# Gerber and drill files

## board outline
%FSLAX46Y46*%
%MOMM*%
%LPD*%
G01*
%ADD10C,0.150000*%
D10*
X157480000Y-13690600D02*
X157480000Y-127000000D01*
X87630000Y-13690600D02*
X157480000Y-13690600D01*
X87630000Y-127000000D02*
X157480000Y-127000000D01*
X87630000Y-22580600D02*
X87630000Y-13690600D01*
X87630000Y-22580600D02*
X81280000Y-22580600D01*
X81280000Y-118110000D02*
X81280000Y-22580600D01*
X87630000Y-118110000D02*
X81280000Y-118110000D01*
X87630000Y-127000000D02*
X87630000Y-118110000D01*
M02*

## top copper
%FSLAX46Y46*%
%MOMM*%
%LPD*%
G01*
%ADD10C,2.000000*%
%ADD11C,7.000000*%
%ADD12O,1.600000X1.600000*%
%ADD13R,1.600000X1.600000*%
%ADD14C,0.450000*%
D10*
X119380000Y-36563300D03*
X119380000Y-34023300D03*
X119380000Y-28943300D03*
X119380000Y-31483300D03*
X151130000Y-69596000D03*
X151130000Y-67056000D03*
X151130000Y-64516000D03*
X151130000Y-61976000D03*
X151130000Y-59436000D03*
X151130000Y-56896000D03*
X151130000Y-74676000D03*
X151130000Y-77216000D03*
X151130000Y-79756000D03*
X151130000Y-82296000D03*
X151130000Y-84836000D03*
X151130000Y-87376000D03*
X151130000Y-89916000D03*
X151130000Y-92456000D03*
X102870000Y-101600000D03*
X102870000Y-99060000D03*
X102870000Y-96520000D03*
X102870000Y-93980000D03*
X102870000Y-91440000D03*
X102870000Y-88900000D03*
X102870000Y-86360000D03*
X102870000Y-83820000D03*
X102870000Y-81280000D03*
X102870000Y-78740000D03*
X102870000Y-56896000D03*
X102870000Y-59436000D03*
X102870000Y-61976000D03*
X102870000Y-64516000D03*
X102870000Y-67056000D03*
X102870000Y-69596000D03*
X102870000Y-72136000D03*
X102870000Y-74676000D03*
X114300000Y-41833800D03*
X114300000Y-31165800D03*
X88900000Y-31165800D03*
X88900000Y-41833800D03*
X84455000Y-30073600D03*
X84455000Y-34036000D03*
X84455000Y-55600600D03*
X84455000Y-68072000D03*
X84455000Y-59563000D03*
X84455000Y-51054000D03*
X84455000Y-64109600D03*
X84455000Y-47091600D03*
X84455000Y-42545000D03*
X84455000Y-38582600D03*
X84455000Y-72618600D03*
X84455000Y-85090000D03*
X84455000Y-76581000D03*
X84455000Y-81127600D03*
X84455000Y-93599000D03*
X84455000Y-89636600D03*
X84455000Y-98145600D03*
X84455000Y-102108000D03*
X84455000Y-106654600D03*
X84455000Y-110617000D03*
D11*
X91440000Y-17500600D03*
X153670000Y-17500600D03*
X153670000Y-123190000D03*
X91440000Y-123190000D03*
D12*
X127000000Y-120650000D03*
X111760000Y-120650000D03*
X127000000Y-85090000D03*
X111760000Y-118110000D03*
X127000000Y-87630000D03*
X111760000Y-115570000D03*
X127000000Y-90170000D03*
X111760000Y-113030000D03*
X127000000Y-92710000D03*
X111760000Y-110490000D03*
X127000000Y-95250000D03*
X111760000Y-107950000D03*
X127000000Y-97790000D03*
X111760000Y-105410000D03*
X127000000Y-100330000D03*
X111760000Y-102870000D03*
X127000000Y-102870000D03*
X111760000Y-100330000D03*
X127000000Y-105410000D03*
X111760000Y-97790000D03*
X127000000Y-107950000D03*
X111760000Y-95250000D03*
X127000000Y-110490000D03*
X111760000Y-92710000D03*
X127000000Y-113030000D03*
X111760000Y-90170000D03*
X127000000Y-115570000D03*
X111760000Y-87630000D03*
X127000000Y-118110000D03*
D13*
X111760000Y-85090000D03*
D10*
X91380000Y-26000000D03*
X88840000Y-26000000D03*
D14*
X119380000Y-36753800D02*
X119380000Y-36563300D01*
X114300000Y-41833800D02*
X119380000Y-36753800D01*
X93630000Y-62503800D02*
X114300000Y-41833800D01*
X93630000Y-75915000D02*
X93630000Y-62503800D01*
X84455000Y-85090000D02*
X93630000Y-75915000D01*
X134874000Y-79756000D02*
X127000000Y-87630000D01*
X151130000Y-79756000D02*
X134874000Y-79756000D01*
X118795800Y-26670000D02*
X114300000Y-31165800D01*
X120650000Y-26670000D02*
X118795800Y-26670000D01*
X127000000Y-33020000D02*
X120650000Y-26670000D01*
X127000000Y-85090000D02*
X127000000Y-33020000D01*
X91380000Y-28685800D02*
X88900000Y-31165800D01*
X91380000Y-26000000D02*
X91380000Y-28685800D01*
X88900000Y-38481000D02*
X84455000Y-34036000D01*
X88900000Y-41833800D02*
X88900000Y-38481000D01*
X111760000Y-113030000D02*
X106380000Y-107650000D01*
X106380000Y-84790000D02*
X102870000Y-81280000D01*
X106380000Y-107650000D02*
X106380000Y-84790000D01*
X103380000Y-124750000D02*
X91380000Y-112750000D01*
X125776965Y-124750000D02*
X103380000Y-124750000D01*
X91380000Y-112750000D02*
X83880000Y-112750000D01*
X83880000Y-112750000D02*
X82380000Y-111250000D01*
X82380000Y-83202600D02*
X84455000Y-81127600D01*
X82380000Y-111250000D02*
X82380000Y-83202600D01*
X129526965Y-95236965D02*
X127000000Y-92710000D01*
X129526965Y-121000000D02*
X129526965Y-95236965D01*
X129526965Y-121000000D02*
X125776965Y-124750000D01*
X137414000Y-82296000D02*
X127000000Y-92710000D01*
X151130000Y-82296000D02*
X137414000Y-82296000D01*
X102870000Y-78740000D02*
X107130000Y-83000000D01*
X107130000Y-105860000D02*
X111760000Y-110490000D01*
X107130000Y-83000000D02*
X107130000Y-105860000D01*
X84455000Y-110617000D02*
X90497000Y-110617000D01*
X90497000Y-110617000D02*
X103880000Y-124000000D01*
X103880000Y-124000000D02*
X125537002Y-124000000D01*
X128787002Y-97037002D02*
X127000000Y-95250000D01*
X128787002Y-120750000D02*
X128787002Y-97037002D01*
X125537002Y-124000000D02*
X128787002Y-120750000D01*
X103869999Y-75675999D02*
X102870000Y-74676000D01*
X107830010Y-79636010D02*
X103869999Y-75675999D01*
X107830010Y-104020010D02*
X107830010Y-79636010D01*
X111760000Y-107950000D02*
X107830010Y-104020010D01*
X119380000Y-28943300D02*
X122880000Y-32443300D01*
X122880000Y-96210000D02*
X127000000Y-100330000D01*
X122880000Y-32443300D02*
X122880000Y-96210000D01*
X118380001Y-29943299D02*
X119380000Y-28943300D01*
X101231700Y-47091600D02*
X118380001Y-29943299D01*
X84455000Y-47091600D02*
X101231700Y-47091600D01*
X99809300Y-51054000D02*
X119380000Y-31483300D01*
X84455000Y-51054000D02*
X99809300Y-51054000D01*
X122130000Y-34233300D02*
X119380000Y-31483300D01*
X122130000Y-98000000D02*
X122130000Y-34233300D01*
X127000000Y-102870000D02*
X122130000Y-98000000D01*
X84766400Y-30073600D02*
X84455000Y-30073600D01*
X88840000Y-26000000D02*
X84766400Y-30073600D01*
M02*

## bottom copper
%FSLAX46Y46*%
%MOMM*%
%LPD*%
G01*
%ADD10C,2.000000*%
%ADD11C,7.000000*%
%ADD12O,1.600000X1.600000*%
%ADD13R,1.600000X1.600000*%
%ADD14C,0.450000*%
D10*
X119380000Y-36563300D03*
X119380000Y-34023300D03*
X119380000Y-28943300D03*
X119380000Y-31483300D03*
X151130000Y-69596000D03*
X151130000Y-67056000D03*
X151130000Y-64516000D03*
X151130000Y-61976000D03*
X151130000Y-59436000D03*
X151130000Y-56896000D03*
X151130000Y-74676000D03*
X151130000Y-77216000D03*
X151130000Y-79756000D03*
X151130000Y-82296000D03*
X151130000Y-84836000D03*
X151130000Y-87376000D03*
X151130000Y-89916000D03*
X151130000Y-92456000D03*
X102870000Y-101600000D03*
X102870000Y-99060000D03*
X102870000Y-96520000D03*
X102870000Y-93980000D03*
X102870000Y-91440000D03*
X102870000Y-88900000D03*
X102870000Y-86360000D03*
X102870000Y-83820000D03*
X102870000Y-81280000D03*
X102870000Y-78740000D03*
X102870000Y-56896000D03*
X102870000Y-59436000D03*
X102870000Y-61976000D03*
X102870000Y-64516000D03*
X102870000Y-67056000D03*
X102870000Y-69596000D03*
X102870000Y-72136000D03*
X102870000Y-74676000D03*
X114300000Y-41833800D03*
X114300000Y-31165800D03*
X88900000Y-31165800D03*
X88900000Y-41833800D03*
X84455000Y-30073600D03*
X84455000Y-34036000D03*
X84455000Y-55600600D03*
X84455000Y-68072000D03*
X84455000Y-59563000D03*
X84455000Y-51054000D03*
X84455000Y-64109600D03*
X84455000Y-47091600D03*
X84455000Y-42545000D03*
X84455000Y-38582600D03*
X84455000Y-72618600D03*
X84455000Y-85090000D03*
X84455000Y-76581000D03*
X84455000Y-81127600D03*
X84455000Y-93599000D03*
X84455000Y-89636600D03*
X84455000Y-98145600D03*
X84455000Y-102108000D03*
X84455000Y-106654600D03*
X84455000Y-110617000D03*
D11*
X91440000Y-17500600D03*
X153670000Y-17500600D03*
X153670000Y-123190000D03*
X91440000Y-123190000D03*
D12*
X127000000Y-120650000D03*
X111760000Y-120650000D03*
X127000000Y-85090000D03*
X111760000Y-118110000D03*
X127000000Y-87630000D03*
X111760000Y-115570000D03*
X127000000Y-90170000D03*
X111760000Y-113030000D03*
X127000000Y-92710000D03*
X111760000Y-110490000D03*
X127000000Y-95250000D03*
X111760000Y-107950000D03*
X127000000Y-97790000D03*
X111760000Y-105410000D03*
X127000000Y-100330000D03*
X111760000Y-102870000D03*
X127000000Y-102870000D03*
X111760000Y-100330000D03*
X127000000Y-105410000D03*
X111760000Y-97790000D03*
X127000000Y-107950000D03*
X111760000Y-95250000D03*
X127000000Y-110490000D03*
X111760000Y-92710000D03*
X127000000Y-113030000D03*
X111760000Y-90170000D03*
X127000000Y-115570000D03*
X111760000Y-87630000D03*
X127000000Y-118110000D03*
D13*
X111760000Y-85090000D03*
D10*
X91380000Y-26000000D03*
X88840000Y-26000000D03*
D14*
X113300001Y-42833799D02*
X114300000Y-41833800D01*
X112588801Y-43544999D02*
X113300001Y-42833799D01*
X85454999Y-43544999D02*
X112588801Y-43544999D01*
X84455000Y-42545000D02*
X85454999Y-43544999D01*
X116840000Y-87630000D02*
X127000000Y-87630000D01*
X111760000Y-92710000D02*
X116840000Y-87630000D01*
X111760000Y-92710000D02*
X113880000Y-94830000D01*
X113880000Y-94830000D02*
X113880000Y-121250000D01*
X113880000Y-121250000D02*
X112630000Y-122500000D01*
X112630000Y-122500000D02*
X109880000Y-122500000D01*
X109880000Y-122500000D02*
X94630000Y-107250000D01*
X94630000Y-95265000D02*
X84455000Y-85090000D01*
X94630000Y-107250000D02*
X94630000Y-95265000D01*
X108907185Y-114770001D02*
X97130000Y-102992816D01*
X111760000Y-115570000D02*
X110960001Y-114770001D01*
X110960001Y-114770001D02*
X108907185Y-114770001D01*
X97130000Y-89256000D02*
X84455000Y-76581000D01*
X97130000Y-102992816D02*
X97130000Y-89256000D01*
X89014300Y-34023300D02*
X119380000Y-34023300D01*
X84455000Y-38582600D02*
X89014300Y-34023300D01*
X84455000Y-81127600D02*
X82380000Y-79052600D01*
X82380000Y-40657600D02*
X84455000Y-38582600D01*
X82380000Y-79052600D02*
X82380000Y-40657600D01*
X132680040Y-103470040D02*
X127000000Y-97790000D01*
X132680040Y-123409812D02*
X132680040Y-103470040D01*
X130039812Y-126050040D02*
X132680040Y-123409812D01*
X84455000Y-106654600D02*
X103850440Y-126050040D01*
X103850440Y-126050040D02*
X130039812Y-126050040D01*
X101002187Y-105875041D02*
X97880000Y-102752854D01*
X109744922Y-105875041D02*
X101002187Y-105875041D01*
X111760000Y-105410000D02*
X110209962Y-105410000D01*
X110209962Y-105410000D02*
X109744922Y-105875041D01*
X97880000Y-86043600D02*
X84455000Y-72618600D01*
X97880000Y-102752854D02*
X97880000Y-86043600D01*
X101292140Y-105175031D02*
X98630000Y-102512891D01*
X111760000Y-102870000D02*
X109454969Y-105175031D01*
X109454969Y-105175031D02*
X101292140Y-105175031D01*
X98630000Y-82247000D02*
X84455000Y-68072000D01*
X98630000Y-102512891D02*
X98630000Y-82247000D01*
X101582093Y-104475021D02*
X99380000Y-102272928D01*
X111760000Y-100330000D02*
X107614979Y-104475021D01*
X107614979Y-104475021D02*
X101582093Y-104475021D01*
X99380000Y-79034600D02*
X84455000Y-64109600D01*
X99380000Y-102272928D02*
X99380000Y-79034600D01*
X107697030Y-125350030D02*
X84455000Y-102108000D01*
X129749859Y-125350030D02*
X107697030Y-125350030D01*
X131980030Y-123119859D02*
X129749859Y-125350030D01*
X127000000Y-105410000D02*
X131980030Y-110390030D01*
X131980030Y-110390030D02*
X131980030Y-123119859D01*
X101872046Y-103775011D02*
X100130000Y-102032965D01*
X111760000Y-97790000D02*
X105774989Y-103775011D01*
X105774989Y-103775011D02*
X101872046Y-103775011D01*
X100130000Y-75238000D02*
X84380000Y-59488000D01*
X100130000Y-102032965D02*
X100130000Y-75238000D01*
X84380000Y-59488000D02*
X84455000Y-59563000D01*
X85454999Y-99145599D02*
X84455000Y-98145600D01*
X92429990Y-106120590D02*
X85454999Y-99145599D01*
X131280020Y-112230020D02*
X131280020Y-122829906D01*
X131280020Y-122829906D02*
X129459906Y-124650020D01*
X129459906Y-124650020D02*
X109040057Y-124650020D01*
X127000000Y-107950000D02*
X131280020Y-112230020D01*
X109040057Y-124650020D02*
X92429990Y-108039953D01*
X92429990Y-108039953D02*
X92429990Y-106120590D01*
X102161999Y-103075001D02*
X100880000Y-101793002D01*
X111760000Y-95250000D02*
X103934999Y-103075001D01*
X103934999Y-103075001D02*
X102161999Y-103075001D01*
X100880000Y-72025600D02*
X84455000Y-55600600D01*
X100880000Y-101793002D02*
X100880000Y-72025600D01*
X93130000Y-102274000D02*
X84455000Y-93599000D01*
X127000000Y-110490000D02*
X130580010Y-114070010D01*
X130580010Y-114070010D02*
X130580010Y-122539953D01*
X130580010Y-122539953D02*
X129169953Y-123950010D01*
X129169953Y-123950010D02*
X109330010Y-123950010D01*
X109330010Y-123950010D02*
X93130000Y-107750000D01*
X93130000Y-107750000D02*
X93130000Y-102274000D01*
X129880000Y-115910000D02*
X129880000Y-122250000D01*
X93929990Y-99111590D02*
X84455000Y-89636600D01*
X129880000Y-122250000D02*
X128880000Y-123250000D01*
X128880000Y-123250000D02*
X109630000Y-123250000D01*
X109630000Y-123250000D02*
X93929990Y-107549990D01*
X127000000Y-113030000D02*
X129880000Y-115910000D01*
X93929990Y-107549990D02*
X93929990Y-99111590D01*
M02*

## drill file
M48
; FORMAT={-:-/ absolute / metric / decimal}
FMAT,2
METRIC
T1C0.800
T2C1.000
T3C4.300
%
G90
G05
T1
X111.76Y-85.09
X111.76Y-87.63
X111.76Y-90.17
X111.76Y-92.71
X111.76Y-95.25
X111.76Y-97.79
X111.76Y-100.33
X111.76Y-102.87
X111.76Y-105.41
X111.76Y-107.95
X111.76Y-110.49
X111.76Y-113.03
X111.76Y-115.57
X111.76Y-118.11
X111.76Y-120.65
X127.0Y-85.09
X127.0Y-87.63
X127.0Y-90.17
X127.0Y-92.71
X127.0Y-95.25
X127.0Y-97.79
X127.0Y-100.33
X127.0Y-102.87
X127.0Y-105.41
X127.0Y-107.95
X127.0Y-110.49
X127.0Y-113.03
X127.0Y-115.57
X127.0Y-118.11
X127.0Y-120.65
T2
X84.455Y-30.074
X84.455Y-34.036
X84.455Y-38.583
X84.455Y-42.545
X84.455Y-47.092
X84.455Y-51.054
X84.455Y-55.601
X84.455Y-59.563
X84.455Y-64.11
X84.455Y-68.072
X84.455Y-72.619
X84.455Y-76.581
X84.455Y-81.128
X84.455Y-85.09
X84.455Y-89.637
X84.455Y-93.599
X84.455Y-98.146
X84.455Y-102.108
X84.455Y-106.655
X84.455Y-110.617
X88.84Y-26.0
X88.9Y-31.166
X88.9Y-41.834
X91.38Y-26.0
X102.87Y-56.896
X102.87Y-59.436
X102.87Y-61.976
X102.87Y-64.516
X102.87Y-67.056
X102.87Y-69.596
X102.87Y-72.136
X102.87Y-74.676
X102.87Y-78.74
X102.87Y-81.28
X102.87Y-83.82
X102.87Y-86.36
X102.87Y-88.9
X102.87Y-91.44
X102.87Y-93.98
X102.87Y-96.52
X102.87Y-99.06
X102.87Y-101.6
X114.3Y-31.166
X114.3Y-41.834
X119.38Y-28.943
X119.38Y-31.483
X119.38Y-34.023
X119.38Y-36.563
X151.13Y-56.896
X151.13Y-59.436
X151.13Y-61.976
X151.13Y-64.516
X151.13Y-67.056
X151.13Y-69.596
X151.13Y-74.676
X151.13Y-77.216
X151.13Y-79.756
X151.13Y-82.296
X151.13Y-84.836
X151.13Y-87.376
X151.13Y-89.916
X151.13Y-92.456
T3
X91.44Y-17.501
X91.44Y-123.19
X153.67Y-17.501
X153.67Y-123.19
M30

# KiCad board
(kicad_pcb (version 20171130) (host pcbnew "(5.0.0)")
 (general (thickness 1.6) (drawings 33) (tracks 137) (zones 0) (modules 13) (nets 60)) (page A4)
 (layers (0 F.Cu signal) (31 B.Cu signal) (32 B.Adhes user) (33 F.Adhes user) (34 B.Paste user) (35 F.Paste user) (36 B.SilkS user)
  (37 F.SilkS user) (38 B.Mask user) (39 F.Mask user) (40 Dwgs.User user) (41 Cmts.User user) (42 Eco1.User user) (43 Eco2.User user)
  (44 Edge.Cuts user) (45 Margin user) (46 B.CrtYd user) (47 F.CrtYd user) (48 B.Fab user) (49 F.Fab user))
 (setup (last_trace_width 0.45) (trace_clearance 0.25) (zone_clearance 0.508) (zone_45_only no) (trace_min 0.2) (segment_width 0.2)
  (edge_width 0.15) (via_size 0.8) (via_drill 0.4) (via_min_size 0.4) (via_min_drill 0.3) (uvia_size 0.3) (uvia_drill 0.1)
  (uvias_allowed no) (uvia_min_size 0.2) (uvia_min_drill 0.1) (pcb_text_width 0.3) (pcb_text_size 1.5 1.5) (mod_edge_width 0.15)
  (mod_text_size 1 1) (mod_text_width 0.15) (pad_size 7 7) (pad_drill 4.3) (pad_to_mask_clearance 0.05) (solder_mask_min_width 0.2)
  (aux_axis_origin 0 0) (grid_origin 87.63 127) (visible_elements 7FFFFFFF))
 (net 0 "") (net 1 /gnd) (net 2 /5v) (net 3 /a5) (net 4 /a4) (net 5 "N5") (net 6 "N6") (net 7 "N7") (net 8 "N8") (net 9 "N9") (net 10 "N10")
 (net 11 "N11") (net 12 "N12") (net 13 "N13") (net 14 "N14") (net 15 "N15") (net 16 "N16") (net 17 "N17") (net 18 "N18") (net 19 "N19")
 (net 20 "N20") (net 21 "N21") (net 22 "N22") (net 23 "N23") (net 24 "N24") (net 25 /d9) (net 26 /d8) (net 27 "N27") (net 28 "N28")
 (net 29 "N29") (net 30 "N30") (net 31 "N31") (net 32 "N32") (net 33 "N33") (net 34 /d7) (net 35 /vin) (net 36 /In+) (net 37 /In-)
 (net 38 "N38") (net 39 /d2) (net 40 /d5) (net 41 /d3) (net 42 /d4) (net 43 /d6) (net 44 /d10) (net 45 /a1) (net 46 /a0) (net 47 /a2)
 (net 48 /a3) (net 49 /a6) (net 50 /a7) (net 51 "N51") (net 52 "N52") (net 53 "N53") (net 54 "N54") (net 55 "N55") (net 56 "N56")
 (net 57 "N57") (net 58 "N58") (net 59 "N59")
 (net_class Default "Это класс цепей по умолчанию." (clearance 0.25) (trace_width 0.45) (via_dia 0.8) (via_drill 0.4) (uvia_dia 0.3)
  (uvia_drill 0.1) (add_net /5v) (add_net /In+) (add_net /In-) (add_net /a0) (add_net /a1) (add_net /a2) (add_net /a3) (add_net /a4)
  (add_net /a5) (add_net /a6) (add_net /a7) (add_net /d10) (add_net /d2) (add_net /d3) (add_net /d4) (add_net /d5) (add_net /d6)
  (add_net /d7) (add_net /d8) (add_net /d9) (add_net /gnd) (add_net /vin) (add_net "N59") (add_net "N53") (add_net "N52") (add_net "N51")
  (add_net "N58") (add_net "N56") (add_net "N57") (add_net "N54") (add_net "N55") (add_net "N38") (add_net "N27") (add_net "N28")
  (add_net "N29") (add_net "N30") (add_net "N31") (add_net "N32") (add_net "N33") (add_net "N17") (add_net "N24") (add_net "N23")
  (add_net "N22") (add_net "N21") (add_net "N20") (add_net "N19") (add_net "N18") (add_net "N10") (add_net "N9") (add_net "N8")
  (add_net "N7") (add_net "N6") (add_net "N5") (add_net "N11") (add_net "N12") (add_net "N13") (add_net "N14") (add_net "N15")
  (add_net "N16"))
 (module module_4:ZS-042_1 (layer F.Cu) (at 119.38 36.5633)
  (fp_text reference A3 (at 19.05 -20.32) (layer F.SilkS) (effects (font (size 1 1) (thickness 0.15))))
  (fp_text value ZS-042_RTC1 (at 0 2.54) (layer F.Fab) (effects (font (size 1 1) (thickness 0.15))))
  (pad 6 thru_hole circle (at 0 0) (size 2 2) (drill 1) (layers *.Cu *.Mask) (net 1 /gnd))
  (pad 5 thru_hole circle (at 0 -2.54) (size 2 2) (drill 1) (layers *.Cu *.Mask) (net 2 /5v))
  (pad 3 thru_hole circle (at 0 -7.62) (size 2 2) (drill 1) (layers *.Cu *.Mask) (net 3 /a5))
  (pad 4 thru_hole circle (at 0 -5.08) (size 2 2) (drill 1) (layers *.Cu *.Mask) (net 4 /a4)))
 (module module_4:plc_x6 (layer F.Cu) (at 151.13 69.596)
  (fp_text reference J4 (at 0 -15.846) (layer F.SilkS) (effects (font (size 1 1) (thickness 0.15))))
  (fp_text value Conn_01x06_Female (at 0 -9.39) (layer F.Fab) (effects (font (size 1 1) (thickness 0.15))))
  (pad 6 thru_hole circle (at 0 0) (size 2 2) (drill 1) (layers *.Cu *.Mask) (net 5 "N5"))
  (pad 5 thru_hole circle (at 0 -2.54) (size 2 2) (drill 1) (layers *.Cu *.Mask) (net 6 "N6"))
  (pad 4 thru_hole circle (at 0 -5.08) (size 2 2) (drill 1) (layers *.Cu *.Mask) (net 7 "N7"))
  (pad 3 thru_hole circle (at 0 -7.62) (size 2 2) (drill 1) (layers *.Cu *.Mask) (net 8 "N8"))
  (pad 2 thru_hole circle (at 0 -10.16) (size 2 2) (drill 1) (layers *.Cu *.Mask) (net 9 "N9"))
  (pad 1 thru_hole circle (at 0 -12.7) (size 2 2) (drill 1) (layers *.Cu *.Mask) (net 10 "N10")))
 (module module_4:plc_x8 (layer F.Cu) (at 151.13 92.456)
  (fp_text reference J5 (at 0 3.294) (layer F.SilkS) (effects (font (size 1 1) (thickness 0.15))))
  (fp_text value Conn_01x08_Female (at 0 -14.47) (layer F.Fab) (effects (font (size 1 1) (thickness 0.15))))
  (pad 1 thru_hole circle (at 0 -17.78) (size 2 2) (drill 1) (layers *.Cu *.Mask) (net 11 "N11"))
  (pad 2 thru_hole circle (at 0 -15.24) (size 2 2) (drill 1) (layers *.Cu *.Mask) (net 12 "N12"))
  (pad 3 thru_hole circle (at 0 -12.7) (size 2 2) (drill 1) (layers *.Cu *.Mask) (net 1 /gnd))
  (pad 4 thru_hole circle (at 0 -10.16) (size 2 2) (drill 1) (layers *.Cu *.Mask) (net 2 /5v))
  (pad 5 thru_hole circle (at 0 -7.62) (size 2 2) (drill 1) (layers *.Cu *.Mask) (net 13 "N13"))
  (pad 6 thru_hole circle (at 0 -5.08) (size 2 2) (drill 1) (layers *.Cu *.Mask) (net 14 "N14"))
  (pad 7 thru_hole circle (at 0 -2.54) (size 2 2) (drill 1) (layers *.Cu *.Mask) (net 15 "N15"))
  (pad 8 thru_hole circle (at 0 0) (size 2 2) (drill 1) (layers *.Cu *.Mask) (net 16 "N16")))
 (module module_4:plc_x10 (layer F.Cu) (at 102.87 101.6)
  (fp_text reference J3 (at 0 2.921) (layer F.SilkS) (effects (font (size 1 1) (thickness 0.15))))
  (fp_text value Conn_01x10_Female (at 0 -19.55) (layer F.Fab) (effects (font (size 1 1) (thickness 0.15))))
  (pad 10 thru_hole circle (at 0 0) (size 2 2) (drill 1) (layers *.Cu *.Mask) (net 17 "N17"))
  (pad 9 thru_hole circle (at 0 -2.54) (size 2 2) (drill 1) (layers *.Cu *.Mask) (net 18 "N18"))
  (pad 8 thru_hole circle (at 0 -5.08) (size 2 2) (drill 1) (layers *.Cu *.Mask) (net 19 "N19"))
  (pad 7 thru_hole circle (at 0 -7.62) (size 2 2) (drill 1) (layers *.Cu *.Mask) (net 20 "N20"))
  (pad 6 thru_hole circle (at 0 -10.16) (size 2 2) (drill 1) (layers *.Cu *.Mask) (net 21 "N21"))
  (pad 5 thru_hole circle (at 0 -12.7) (size 2 2) (drill 1) (layers *.Cu *.Mask) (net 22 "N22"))
  (pad 4 thru_hole circle (at 0 -15.24) (size 2 2) (drill 1) (layers *.Cu *.Mask) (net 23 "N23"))
  (pad 3 thru_hole circle (at 0 -17.78) (size 2 2) (drill 1) (layers *.Cu *.Mask) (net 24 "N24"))
  (pad 2 thru_hole circle (at 0 -20.32) (size 2 2) (drill 1) (layers *.Cu *.Mask) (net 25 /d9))
  (pad 1 thru_hole circle (at 0 -22.86) (size 2 2) (drill 1) (layers *.Cu *.Mask) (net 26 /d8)))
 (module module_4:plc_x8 (layer F.Cu) (at 102.87 74.676)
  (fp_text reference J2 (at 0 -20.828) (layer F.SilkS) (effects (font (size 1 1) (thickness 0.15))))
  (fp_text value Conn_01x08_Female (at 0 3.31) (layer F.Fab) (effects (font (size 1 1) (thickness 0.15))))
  (pad 1 thru_hole circle (at 0 -17.78) (size 2 2) (drill 1) (layers *.Cu *.Mask) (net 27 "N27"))
  (pad 2 thru_hole circle (at 0 -15.24) (size 2 2) (drill 1) (layers *.Cu *.Mask) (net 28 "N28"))
  (pad 3 thru_hole circle (at 0 -12.7) (size 2 2) (drill 1) (layers *.Cu *.Mask) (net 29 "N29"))
  (pad 4 thru_hole circle (at 0 -10.16) (size 2 2) (drill 1) (layers *.Cu *.Mask) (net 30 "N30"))
  (pad 5 thru_hole circle (at 0 -7.62) (size 2 2) (drill 1) (layers *.Cu *.Mask) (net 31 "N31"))
  (pad 6 thru_hole circle (at 0 -5.08) (size 2 2) (drill 1) (layers *.Cu *.Mask) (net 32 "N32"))
  (pad 7 thru_hole circle (at 0 -2.54) (size 2 2) (drill 1) (layers *.Cu *.Mask) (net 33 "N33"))
  (pad 8 thru_hole circle (at 0 0) (size 2 2) (drill 1) (layers *.Cu *.Mask) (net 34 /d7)))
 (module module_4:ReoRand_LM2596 (layer F.Cu) (at 88.9 41.8338)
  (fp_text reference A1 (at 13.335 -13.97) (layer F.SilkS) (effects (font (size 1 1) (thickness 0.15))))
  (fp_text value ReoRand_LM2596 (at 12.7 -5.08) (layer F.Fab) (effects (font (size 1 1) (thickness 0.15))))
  (pad 4 thru_hole circle (at 25.4 0) (size 2 2) (drill 1) (layers *.Cu *.Mask) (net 1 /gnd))
  (pad 3 thru_hole circle (at 25.4 -10.668) (size 2 2) (drill 1) (layers *.Cu *.Mask) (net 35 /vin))
  (pad 1 thru_hole circle (at 0 -10.668) (size 2 2) (drill 1) (layers *.Cu *.Mask) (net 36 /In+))
  (pad 2 thru_hole circle (at 0 0) (size 2 2) (drill 1) (layers *.Cu *.Mask) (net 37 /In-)))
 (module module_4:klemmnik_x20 (layer F.Cu) (at 84.455 110.617)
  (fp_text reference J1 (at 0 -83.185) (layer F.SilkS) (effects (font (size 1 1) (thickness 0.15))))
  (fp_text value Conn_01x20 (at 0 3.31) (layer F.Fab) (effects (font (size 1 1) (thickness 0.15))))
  (pad 1 thru_hole circle (at 0 -80.5434) (size 2 2) (drill 1) (layers *.Cu *.Mask) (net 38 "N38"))
  (pad 2 thru_hole circle (at 0 -76.581) (size 2 2) (drill 1) (layers *.Cu *.Mask) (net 37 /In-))
  (pad 7 thru_hole circle (at 0 -55.0164) (size 2 2) (drill 1) (layers *.Cu *.Mask) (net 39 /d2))
  (pad 10 thru_hole circle (at 0 -42.545) (size 2 2) (drill 1) (layers *.Cu *.Mask) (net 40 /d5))
  (pad 8 thru_hole circle (at 0 -51.054) (size 2 2) (drill 1) (layers *.Cu *.Mask) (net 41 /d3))
  (pad 6 thru_hole circle (at 0 -59.563) (size 2 2) (drill 1) (layers *.Cu *.Mask) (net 4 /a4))
  (pad 9 thru_hole circle (at 0 -46.5074) (size 2 2) (drill 1) (layers *.Cu *.Mask) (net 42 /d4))
  (pad 5 thru_hole circle (at 0 -63.5254) (size 2 2) (drill 1) (layers *.Cu *.Mask) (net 3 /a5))
  (pad 4 thru_hole circle (at 0 -68.072) (size 2 2) (drill 1) (layers *.Cu *.Mask) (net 1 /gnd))
  (pad 3 thru_hole circle (at 0 -72.0344) (size 2 2) (drill 1) (layers *.Cu *.Mask) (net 2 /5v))
  (pad 11 thru_hole circle (at 0 -37.9984) (size 2 2) (drill 1) (layers *.Cu *.Mask) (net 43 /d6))
  (pad 14 thru_hole circle (at 0 -25.527) (size 2 2) (drill 1) (layers *.Cu *.Mask) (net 1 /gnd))
  (pad 12 thru_hole circle (at 0 -34.036) (size 2 2) (drill 1) (layers *.Cu *.Mask) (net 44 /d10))
  (pad 13 thru_hole circle (at 0 -29.4894) (size 2 2) (drill 1) (layers *.Cu *.Mask) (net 2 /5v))
  (pad 16 thru_hole circle (at 0 -17.018) (size 2 2) (drill 1) (layers *.Cu *.Mask) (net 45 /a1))
  (pad 15 thru_hole circle (at 0 -20.9804) (size 2 2) (drill 1) (layers *.Cu *.Mask) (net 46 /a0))
  (pad 17 thru_hole circle (at 0 -12.4714) (size 2 2) (drill 1) (layers *.Cu *.Mask) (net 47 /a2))
  (pad 18 thru_hole circle (at 0 -8.509) (size 2 2) (drill 1) (layers *.Cu *.Mask) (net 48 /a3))
  (pad 19 thru_hole circle (at 0 -3.9624) (size 2 2) (drill 1) (layers *.Cu *.Mask) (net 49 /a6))
  (pad 20 thru_hole circle (at 0 0) (size 2 2) (drill 1) (layers *.Cu *.Mask) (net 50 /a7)))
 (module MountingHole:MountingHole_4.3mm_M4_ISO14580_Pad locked (layer F.Cu) (at 91.44 17.5006)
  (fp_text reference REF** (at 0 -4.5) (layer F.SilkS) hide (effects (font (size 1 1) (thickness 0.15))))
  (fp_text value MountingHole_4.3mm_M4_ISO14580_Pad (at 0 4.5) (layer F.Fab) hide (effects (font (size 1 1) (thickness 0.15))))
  (pad "" thru_hole circle (at 0 0) (size 7 7) (drill 4.3) (layers *.Cu *.Mask)))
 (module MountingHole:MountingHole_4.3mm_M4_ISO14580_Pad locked (layer F.Cu) (at 153.67 17.5006)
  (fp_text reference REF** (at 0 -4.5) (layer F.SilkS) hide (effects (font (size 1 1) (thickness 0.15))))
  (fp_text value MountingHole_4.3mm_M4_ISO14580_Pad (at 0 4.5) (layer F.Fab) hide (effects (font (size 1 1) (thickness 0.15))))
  (pad "" thru_hole circle (at 0 0) (size 7 7) (drill 4.3) (layers *.Cu *.Mask)))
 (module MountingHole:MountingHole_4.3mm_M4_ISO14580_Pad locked (layer F.Cu) (at 153.67 123.19)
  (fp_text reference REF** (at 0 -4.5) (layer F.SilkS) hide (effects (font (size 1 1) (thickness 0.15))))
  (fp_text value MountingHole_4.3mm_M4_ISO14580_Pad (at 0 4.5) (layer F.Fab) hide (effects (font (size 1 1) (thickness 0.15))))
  (pad "" thru_hole circle (at 0 0) (size 7 7) (drill 4.3) (layers *.Cu *.Mask)))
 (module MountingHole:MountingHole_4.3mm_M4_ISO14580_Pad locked (layer F.Cu) (at 91.44 123.19)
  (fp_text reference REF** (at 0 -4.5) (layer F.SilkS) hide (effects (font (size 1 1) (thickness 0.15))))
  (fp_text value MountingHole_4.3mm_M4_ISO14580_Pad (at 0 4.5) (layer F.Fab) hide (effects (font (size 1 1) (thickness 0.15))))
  (pad "" thru_hole circle (at 0 0) (size 7 7) (drill 4.3) (layers *.Cu *.Mask)))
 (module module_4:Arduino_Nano (layer F.Cu) (at 111.76 85.09)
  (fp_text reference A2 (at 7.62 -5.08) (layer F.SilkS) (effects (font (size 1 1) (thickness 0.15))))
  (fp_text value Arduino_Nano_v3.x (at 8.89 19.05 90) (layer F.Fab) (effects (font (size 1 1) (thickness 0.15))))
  (pad 16 thru_hole oval (at 15.24 35.56) (size 1.6 1.6) (drill 0.8) (layers *.Cu *.Mask) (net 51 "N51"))
  (pad 15 thru_hole oval (at 0 35.56) (size 1.6 1.6) (drill 0.8) (layers *.Cu *.Mask) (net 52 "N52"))
  (pad 30 thru_hole oval (at 15.24 0) (size 1.6 1.6) (drill 0.8) (layers *.Cu *.Mask) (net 35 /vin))
  (pad 14 thru_hole oval (at 0 33.02) (size 1.6 1.6) (drill 0.8) (layers *.Cu *.Mask) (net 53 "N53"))
  (pad 29 thru_hole oval (at 15.24 2.54) (size 1.6 1.6) (drill 0.8) (layers *.Cu *.Mask) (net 1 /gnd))
  (pad 13 thru_hole oval (at 0 30.48) (size 1.6 1.6) (drill 0.8) (layers *.Cu *.Mask) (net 44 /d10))
  (pad 28 thru_hole oval (at 15.24 5.08) (size 1.6 1.6) (drill 0.8) (layers *.Cu *.Mask) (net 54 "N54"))
  (pad 12 thru_hole oval (at 0 27.94) (size 1.6 1.6) (drill 0.8) (layers *.Cu *.Mask) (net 25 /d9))
  (pad 27 thru_hole oval (at 15.24 7.62) (size 1.6 1.6) (drill 0.8) (layers *.Cu *.Mask) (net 2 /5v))
  (pad 11 thru_hole oval (at 0 25.4) (size 1.6 1.6) (drill 0.8) (layers *.Cu *.Mask) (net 26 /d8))
  (pad 26 thru_hole oval (at 15.24 10.16) (size 1.6 1.6) (drill 0.8) (layers *.Cu *.Mask) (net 50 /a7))
  (pad 10 thru_hole oval (at 0 22.86) (size 1.6 1.6) (drill 0.8) (layers *.Cu *.Mask) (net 34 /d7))
  (pad 25 thru_hole oval (at 15.24 12.7) (size 1.6 1.6) (drill 0.8) (layers *.Cu *.Mask) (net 49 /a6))
  (pad 9 thru_hole oval (at 0 20.32) (size 1.6 1.6) (drill 0.8) (layers *.Cu *.Mask) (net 43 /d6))
  (pad 24 thru_hole oval (at 15.24 15.24) (size 1.6 1.6) (drill 0.8) (layers *.Cu *.Mask) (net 3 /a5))
  (pad 8 thru_hole oval (at 0 17.78) (size 1.6 1.6) (drill 0.8) (layers *.Cu *.Mask) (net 40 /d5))
  (pad 23 thru_hole oval (at 15.24 17.78) (size 1.6 1.6) (drill 0.8) (layers *.Cu *.Mask) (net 4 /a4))
  (pad 7 thru_hole oval (at 0 15.24) (size 1.6 1.6) (drill 0.8) (layers *.Cu *.Mask) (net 42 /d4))
  (pad 22 thru_hole oval (at 15.24 20.32) (size 1.6 1.6) (drill 0.8) (layers *.Cu *.Mask) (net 48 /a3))
  (pad 6 thru_hole oval (at 0 12.7) (size 1.6 1.6) (drill 0.8) (layers *.Cu *.Mask) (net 41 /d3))
  (pad 21 thru_hole oval (at 15.24 22.86) (size 1.6 1.6) (drill 0.8) (layers *.Cu *.Mask) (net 47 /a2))
  (pad 5 thru_hole oval (at 0 10.16) (size 1.6 1.6) (drill 0.8) (layers *.Cu *.Mask) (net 39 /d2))
  (pad 20 thru_hole oval (at 15.24 25.4) (size 1.6 1.6) (drill 0.8) (layers *.Cu *.Mask) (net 45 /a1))
  (pad 4 thru_hole oval (at 0 7.62) (size 1.6 1.6) (drill 0.8) (layers *.Cu *.Mask) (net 1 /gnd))
  (pad 19 thru_hole oval (at 15.24 27.94) (size 1.6 1.6) (drill 0.8) (layers *.Cu *.Mask) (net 46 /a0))
  (pad 3 thru_hole oval (at 0 5.08) (size 1.6 1.6) (drill 0.8) (layers *.Cu *.Mask) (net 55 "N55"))
  (pad 18 thru_hole oval (at 15.24 30.48) (size 1.6 1.6) (drill 0.8) (layers *.Cu *.Mask) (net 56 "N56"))
  (pad 2 thru_hole oval (at 0 2.54) (size 1.6 1.6) (drill 0.8) (layers *.Cu *.Mask) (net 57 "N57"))
  (pad 17 thru_hole oval (at 15.24 33.02) (size 1.6 1.6) (drill 0.8) (layers *.Cu *.Mask) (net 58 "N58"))
  (pad 1 thru_hole rect (at 0 0) (size 1.6 1.6) (drill 0.8) (layers *.Cu *.Mask) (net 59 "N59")))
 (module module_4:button (layer F.Cu) (at 91.38 26 90)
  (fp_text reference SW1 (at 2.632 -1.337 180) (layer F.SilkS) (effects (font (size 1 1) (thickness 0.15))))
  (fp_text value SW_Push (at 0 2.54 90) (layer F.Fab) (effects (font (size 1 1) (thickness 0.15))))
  (pad 2 thru_hole circle (at 0 0 90) (size 2 2) (drill 1) (layers *.Cu *.Mask) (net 36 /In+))
  (pad 1 thru_hole circle (at 0 -2.54 90) (size 2 2) (drill 1) (layers *.Cu *.Mask) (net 38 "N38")))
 (gr_line (start 157.48 13.6906) (end 157.48 127) (layer Edge.Cuts) (width 0.15))
 (gr_line (start 87.63 13.6906) (end 157.48 13.6906) (layer Edge.Cuts) (width 0.15))
 (gr_line (start 87.63 127) (end 157.48 127) (layer Edge.Cuts) (width 0.15))
 (gr_line (start 87.63 22.5806) (end 87.63 13.6906) (layer Edge.Cuts) (width 0.15))
 (gr_line (start 87.63 22.5806) (end 81.28 22.5806) (layer Edge.Cuts) (width 0.15))
 (gr_line (start 81.28 118.11) (end 81.28 22.5806) (layer Edge.Cuts) (width 0.15))
 (gr_line (start 87.63 118.11) (end 81.28 118.11) (layer Edge.Cuts) (width 0.15))
 (gr_line (start 87.63 127) (end 87.63 118.11) (layer Edge.Cuts) (width 0.15))
 (segment (start 113.300001 42.833799) (end 114.3 41.8338) (width 0.45) (layer B.Cu) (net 1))
 (segment (start 112.588801 43.544999) (end 113.300001 42.833799) (width 0.45) (layer B.Cu) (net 1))
 (segment (start 85.454999 43.544999) (end 112.588801 43.544999) (width 0.45) (layer B.Cu) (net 1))
 (segment (start 84.455 42.545) (end 85.454999 43.544999) (width 0.45) (layer B.Cu) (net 1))
 (segment (start 116.84 87.63) (end 127 87.63) (width 0.45) (layer B.Cu) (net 1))
 (segment (start 111.76 92.71) (end 116.84 87.63) (width 0.45) (layer B.Cu) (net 1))
 (segment (start 111.76 92.71) (end 113.88 94.83) (width 0.45) (layer B.Cu) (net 1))
 (segment (start 113.88 94.83) (end 113.88 121.25) (width 0.45) (layer B.Cu) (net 1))
 (segment (start 113.88 121.25) (end 112.63 122.5) (width 0.45) (layer B.Cu) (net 1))
 (segment (start 112.63 122.5) (end 109.88 122.5) (width 0.45) (layer B.Cu) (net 1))
 (segment (start 109.88 122.5) (end 94.63 107.25) (width 0.45) (layer B.Cu) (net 1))
 (segment (start 94.63 95.265) (end 84.455 85.09) (width 0.45) (layer B.Cu) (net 1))
 (segment (start 94.63 107.25) (end 94.63 95.265) (width 0.45) (layer B.Cu) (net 1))
 (segment (start 119.38 36.7538) (end 119.38 36.5633) (width 0.45) (layer F.Cu) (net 1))
 (segment (start 114.3 41.8338) (end 119.38 36.7538) (width 0.45) (layer F.Cu) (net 1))
 (segment (start 93.63 62.5038) (end 114.3 41.8338) (width 0.45) (layer F.Cu) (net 1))
 (segment (start 93.63 75.915) (end 93.63 62.5038) (width 0.45) (layer F.Cu) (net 1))
 (segment (start 84.455 85.09) (end 93.63 75.915) (width 0.45) (layer F.Cu) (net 1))
 (segment (start 134.874 79.756) (end 127 87.63) (width 0.45) (layer F.Cu) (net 1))
 (segment (start 151.13 79.756) (end 134.874 79.756) (width 0.45) (layer F.Cu) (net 1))
 (segment (start 118.7958 26.67) (end 114.3 31.1658) (width 0.45) (layer F.Cu) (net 35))
 (segment (start 120.65 26.67) (end 118.7958 26.67) (width 0.45) (layer F.Cu) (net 35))
 (segment (start 127 33.02) (end 120.65 26.67) (width 0.45) (layer F.Cu) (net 35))
 (segment (start 127 85.09) (end 127 33.02) (width 0.45) (layer F.Cu) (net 35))
 (segment (start 91.38 28.6858) (end 88.9 31.1658) (width 0.45) (layer F.Cu) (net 36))
 (segment (start 91.38 26) (end 91.38 28.6858) (width 0.45) (layer F.Cu) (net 36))
 (segment (start 88.9 38.481) (end 84.455 34.036) (width 0.45) (layer F.Cu) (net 37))
 (segment (start 88.9 41.8338) (end 88.9 38.481) (width 0.45) (layer F.Cu) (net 37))
 (segment (start 108.907185 114.770001) (end 97.13 102.992816) (width 0.45) (layer B.Cu) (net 44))
 (segment (start 111.76 115.57) (end 110.960001 114.770001) (width 0.45) (layer B.Cu) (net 44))
 (segment (start 110.960001 114.770001) (end 108.907185 114.770001) (width 0.45) (layer B.Cu) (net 44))
 (segment (start 97.13 89.256) (end 84.455 76.581) (width 0.45) (layer B.Cu) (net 44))
 (segment (start 97.13 102.992816) (end 97.13 89.256) (width 0.45) (layer B.Cu) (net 44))
 (segment (start 111.76 113.03) (end 106.38 107.65) (width 0.45) (layer F.Cu) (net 25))
 (segment (start 106.38 84.79) (end 102.87 81.28) (width 0.45) (layer F.Cu) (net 25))
 (segment (start 106.38 107.65) (end 106.38 84.79) (width 0.45) (layer F.Cu) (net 25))
 (segment (start 89.0143 34.0233) (end 119.38 34.0233) (width 0.45) (layer B.Cu) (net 2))
 (segment (start 84.455 38.5826) (end 89.0143 34.0233) (width 0.45) (layer B.Cu) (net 2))
 (segment (start 103.38 124.75) (end 91.38 112.75) (width 0.45) (layer F.Cu) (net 2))
 (segment (start 125.776965 124.75) (end 103.38 124.75) (width 0.45) (layer F.Cu) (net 2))
 (segment (start 91.38 112.75) (end 83.88 112.75) (width 0.45) (layer F.Cu) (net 2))
 (segment (start 83.88 112.75) (end 82.38 111.25) (width 0.45) (layer F.Cu) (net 2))
 (segment (start 82.38 83.2026) (end 84.455 81.1276) (width 0.45) (layer F.Cu) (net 2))
 (segment (start 82.38 111.25) (end 82.38 83.2026) (width 0.45) (layer F.Cu) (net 2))
 (segment (start 129.526965 95.236965) (end 127 92.71) (width 0.45) (layer F.Cu) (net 2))
 (segment (start 129.526965 121) (end 129.526965 95.236965) (width 0.45) (layer F.Cu) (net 2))
 (segment (start 129.526965 121) (end 125.776965 124.75) (width 0.45) (layer F.Cu) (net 2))
 (segment (start 137.414 82.296) (end 127 92.71) (width 0.45) (layer F.Cu) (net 2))
 (segment (start 151.13 82.296) (end 137.414 82.296) (width 0.45) (layer F.Cu) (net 2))
 (segment (start 84.455 81.1276) (end 82.38 79.0526) (width 0.45) (layer B.Cu) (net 2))
 (segment (start 82.38 40.6576) (end 84.455 38.5826) (width 0.45) (layer B.Cu) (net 2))
 (segment (start 82.38 79.0526) (end 82.38 40.6576) (width 0.45) (layer B.Cu) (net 2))
 (segment (start 102.87 78.74) (end 107.13 83) (width 0.45) (layer F.Cu) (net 26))
 (segment (start 107.13 105.86) (end 111.76 110.49) (width 0.45) (layer F.Cu) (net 26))
 (segment (start 107.13 83) (end 107.13 105.86) (width 0.45) (layer F.Cu) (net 26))
 (segment (start 84.455 110.617) (end 90.497 110.617) (width 0.45) (layer F.Cu) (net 50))
 (segment (start 90.497 110.617) (end 103.88 124) (width 0.45) (layer F.Cu) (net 50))
 (segment (start 103.88 124) (end 125.537002 124) (width 0.45) (layer F.Cu) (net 50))
 (segment (start 128.787002 97.037002) (end 127 95.25) (width 0.45) (layer F.Cu) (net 50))
 (segment (start 128.787002 120.75) (end 128.787002 97.037002) (width 0.45) (layer F.Cu) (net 50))
 (segment (start 125.537002 124) (end 128.787002 120.75) (width 0.45) (layer F.Cu) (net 50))
 (segment (start 103.869999 75.675999) (end 102.87 74.676) (width 0.45) (layer F.Cu) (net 34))
 (segment (start 107.83001 79.63601) (end 103.869999 75.675999) (width 0.45) (layer F.Cu) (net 34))
 (segment (start 107.83001 104.02001) (end 107.83001 79.63601) (width 0.45) (layer F.Cu) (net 34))
 (segment (start 111.76 107.95) (end 107.83001 104.02001) (width 0.45) (layer F.Cu) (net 34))
 (segment (start 132.68004 103.47004) (end 127 97.79) (width 0.45) (layer B.Cu) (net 49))
 (segment (start 132.68004 123.409812) (end 132.68004 103.47004) (width 0.45) (layer B.Cu) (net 49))
 (segment (start 130.039812 126.05004) (end 132.68004 123.409812) (width 0.45) (layer B.Cu) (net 49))
 (segment (start 84.455 106.6546) (end 103.85044 126.05004) (width 0.45) (layer B.Cu) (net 49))
 (segment (start 103.85044 126.05004) (end 130.039812 126.05004) (width 0.45) (layer B.Cu) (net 49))
 (segment (start 101.002187 105.875041) (end 97.88 102.752854) (width 0.45) (layer B.Cu) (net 43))
 (segment (start 109.744922 105.875041) (end 101.002187 105.875041) (width 0.45) (layer B.Cu) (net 43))
 (segment (start 111.76 105.41) (end 110.209962 105.41) (width 0.45) (layer B.Cu) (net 43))
 (segment (start 110.209962 105.41) (end 109.744922 105.875041) (width 0.45) (layer B.Cu) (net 43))
 (segment (start 97.88 86.0436) (end 84.455 72.6186) (width 0.45) (layer B.Cu) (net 43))
 (segment (start 97.88 102.752854) (end 97.88 86.0436) (width 0.45) (layer B.Cu) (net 43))
 (segment (start 119.38 28.9433) (end 122.88 32.4433) (width 0.45) (layer F.Cu) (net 3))
 (segment (start 122.88 96.21) (end 127 100.33) (width 0.45) (layer F.Cu) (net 3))
 (segment (start 122.88 32.4433) (end 122.88 96.21) (width 0.45) (layer F.Cu) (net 3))
 (segment (start 118.380001 29.943299) (end 119.38 28.9433) (width 0.45) (layer F.Cu) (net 3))
 (segment (start 101.2317 47.0916) (end 118.380001 29.943299) (width 0.45) (layer F.Cu) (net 3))
 (segment (start 84.455 47.0916) (end 101.2317 47.0916) (width 0.45) (layer F.Cu) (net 3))
 (segment (start 101.29214 105.175031) (end 98.63 102.512891) (width 0.45) (layer B.Cu) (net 40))
 (segment (start 111.76 102.87) (end 109.454969 105.175031) (width 0.45) (layer B.Cu) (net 40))
 (segment (start 109.454969 105.175031) (end 101.29214 105.175031) (width 0.45) (layer B.Cu) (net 40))
 (segment (start 98.63 82.247) (end 84.455 68.072) (width 0.45) (layer B.Cu) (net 40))
 (segment (start 98.63 102.512891) (end 98.63 82.247) (width 0.45) (layer B.Cu) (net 40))
 (segment (start 99.8093 51.054) (end 119.38 31.4833) (width 0.45) (layer F.Cu) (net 4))
 (segment (start 84.455 51.054) (end 99.8093 51.054) (width 0.45) (layer F.Cu) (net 4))
 (segment (start 122.13 34.2333) (end 119.38 31.4833) (width 0.45) (layer F.Cu) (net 4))
 (segment (start 122.13 98) (end 122.13 34.2333) (width 0.45) (layer F.Cu) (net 4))
 (segment (start 127 102.87) (end 122.13 98) (width 0.45) (layer F.Cu) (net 4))
 (segment (start 101.582093 104.475021) (end 99.38 102.272928) (width 0.45) (layer B.Cu) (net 42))
 (segment (start 111.76 100.33) (end 107.614979 104.475021) (width 0.45) (layer B.Cu) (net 42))
 (segment (start 107.614979 104.475021) (end 101.582093 104.475021) (width 0.45) (layer B.Cu) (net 42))
 (segment (start 99.38 79.0346) (end 84.455 64.1096) (width 0.45) (layer B.Cu) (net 42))
 (segment (start 99.38 102.272928) (end 99.38 79.0346) (width 0.45) (layer B.Cu) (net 42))
 (segment (start 107.69703 125.35003) (end 84.455 102.108) (width 0.45) (layer B.Cu) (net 48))
 (segment (start 129.749859 125.35003) (end 107.69703 125.35003) (width 0.45) (layer B.Cu) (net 48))
 (segment (start 131.98003 123.119859) (end 129.749859 125.35003) (width 0.45) (layer B.Cu) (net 48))
 (segment (start 127 105.41) (end 131.98003 110.39003) (width 0.45) (layer B.Cu) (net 48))
 (segment (start 131.98003 110.39003) (end 131.98003 123.119859) (width 0.45) (layer B.Cu) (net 48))
 (segment (start 101.872046 103.775011) (end 100.13 102.032965) (width 0.45) (layer B.Cu) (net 41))
 (segment (start 111.76 97.79) (end 105.774989 103.775011) (width 0.45) (layer B.Cu) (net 41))
 (segment (start 105.774989 103.775011) (end 101.872046 103.775011) (width 0.45) (layer B.Cu) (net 41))
 (segment (start 100.13 75.238) (end 84.38 59.488) (width 0.45) (layer B.Cu) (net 41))
 (segment (start 100.13 102.032965) (end 100.13 75.238) (width 0.45) (layer B.Cu) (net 41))
 (segment (start 84.38 59.488) (end 84.455 59.563) (width 0.45) (layer B.Cu) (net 41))
 (segment (start 85.454999 99.145599) (end 84.455 98.1456) (width 0.45) (layer B.Cu) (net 47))
 (segment (start 92.42999 106.12059) (end 85.454999 99.145599) (width 0.45) (layer B.Cu) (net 47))
 (segment (start 131.28002 112.23002) (end 131.28002 122.829906) (width 0.45) (layer B.Cu) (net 47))
 (segment (start 131.28002 122.829906) (end 129.459906 124.65002) (width 0.45) (layer B.Cu) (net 47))
 (segment (start 129.459906 124.65002) (end 109.040057 124.65002) (width 0.45) (layer B.Cu) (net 47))
 (segment (start 127 107.95) (end 131.28002 112.23002) (width 0.45) (layer B.Cu) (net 47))
 (segment (start 109.040057 124.65002) (end 92.42999 108.039953) (width 0.45) (layer B.Cu) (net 47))
 (segment (start 92.42999 108.039953) (end 92.42999 106.12059) (width 0.45) (layer B.Cu) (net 47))
 (segment (start 102.161999 103.075001) (end 100.88 101.793002) (width 0.45) (layer B.Cu) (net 39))
 (segment (start 111.76 95.25) (end 103.934999 103.075001) (width 0.45) (layer B.Cu) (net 39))
 (segment (start 103.934999 103.075001) (end 102.161999 103.075001) (width 0.45) (layer B.Cu) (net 39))
 (segment (start 100.88 72.0256) (end 84.455 55.6006) (width 0.45) (layer B.Cu) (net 39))
 (segment (start 100.88 101.793002) (end 100.88 72.0256) (width 0.45) (layer B.Cu) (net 39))
 (segment (start 93.13 102.274) (end 84.455 93.599) (width 0.45) (layer B.Cu) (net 45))
 (segment (start 127 110.49) (end 130.58001 114.07001) (width 0.45) (layer B.Cu) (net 45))
 (segment (start 130.58001 114.07001) (end 130.58001 122.539953) (width 0.45) (layer B.Cu) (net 45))
 (segment (start 130.58001 122.539953) (end 129.169953 123.95001) (width 0.45) (layer B.Cu) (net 45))
 (segment (start 129.169953 123.95001) (end 109.33001 123.95001) (width 0.45) (layer B.Cu) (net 45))
 (segment (start 109.33001 123.95001) (end 93.13 107.75) (width 0.45) (layer B.Cu) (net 45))
 (segment (start 93.13 107.75) (end 93.13 102.274) (width 0.45) (layer B.Cu) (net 45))
 (segment (start 129.88 115.91) (end 129.88 122.25) (width 0.45) (layer B.Cu) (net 46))
 (segment (start 93.92999 99.11159) (end 84.455 89.6366) (width 0.45) (layer B.Cu) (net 46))
 (segment (start 129.88 122.25) (end 128.88 123.25) (width 0.45) (layer B.Cu) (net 46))
 (segment (start 128.88 123.25) (end 109.63 123.25) (width 0.45) (layer B.Cu) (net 46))
 (segment (start 109.63 123.25) (end 93.92999 107.54999) (width 0.45) (layer B.Cu) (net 46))
 (segment (start 127 113.03) (end 129.88 115.91) (width 0.45) (layer B.Cu) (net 46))
 (segment (start 93.92999 107.54999) (end 93.92999 99.11159) (width 0.45) (layer B.Cu) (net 46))
 (segment (start 84.7664 30.0736) (end 84.455 30.0736) (width 0.45) (layer F.Cu) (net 38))
 (segment (start 88.84 26) (end 84.7664 30.0736) (width 0.45) (layer F.Cu) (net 38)))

